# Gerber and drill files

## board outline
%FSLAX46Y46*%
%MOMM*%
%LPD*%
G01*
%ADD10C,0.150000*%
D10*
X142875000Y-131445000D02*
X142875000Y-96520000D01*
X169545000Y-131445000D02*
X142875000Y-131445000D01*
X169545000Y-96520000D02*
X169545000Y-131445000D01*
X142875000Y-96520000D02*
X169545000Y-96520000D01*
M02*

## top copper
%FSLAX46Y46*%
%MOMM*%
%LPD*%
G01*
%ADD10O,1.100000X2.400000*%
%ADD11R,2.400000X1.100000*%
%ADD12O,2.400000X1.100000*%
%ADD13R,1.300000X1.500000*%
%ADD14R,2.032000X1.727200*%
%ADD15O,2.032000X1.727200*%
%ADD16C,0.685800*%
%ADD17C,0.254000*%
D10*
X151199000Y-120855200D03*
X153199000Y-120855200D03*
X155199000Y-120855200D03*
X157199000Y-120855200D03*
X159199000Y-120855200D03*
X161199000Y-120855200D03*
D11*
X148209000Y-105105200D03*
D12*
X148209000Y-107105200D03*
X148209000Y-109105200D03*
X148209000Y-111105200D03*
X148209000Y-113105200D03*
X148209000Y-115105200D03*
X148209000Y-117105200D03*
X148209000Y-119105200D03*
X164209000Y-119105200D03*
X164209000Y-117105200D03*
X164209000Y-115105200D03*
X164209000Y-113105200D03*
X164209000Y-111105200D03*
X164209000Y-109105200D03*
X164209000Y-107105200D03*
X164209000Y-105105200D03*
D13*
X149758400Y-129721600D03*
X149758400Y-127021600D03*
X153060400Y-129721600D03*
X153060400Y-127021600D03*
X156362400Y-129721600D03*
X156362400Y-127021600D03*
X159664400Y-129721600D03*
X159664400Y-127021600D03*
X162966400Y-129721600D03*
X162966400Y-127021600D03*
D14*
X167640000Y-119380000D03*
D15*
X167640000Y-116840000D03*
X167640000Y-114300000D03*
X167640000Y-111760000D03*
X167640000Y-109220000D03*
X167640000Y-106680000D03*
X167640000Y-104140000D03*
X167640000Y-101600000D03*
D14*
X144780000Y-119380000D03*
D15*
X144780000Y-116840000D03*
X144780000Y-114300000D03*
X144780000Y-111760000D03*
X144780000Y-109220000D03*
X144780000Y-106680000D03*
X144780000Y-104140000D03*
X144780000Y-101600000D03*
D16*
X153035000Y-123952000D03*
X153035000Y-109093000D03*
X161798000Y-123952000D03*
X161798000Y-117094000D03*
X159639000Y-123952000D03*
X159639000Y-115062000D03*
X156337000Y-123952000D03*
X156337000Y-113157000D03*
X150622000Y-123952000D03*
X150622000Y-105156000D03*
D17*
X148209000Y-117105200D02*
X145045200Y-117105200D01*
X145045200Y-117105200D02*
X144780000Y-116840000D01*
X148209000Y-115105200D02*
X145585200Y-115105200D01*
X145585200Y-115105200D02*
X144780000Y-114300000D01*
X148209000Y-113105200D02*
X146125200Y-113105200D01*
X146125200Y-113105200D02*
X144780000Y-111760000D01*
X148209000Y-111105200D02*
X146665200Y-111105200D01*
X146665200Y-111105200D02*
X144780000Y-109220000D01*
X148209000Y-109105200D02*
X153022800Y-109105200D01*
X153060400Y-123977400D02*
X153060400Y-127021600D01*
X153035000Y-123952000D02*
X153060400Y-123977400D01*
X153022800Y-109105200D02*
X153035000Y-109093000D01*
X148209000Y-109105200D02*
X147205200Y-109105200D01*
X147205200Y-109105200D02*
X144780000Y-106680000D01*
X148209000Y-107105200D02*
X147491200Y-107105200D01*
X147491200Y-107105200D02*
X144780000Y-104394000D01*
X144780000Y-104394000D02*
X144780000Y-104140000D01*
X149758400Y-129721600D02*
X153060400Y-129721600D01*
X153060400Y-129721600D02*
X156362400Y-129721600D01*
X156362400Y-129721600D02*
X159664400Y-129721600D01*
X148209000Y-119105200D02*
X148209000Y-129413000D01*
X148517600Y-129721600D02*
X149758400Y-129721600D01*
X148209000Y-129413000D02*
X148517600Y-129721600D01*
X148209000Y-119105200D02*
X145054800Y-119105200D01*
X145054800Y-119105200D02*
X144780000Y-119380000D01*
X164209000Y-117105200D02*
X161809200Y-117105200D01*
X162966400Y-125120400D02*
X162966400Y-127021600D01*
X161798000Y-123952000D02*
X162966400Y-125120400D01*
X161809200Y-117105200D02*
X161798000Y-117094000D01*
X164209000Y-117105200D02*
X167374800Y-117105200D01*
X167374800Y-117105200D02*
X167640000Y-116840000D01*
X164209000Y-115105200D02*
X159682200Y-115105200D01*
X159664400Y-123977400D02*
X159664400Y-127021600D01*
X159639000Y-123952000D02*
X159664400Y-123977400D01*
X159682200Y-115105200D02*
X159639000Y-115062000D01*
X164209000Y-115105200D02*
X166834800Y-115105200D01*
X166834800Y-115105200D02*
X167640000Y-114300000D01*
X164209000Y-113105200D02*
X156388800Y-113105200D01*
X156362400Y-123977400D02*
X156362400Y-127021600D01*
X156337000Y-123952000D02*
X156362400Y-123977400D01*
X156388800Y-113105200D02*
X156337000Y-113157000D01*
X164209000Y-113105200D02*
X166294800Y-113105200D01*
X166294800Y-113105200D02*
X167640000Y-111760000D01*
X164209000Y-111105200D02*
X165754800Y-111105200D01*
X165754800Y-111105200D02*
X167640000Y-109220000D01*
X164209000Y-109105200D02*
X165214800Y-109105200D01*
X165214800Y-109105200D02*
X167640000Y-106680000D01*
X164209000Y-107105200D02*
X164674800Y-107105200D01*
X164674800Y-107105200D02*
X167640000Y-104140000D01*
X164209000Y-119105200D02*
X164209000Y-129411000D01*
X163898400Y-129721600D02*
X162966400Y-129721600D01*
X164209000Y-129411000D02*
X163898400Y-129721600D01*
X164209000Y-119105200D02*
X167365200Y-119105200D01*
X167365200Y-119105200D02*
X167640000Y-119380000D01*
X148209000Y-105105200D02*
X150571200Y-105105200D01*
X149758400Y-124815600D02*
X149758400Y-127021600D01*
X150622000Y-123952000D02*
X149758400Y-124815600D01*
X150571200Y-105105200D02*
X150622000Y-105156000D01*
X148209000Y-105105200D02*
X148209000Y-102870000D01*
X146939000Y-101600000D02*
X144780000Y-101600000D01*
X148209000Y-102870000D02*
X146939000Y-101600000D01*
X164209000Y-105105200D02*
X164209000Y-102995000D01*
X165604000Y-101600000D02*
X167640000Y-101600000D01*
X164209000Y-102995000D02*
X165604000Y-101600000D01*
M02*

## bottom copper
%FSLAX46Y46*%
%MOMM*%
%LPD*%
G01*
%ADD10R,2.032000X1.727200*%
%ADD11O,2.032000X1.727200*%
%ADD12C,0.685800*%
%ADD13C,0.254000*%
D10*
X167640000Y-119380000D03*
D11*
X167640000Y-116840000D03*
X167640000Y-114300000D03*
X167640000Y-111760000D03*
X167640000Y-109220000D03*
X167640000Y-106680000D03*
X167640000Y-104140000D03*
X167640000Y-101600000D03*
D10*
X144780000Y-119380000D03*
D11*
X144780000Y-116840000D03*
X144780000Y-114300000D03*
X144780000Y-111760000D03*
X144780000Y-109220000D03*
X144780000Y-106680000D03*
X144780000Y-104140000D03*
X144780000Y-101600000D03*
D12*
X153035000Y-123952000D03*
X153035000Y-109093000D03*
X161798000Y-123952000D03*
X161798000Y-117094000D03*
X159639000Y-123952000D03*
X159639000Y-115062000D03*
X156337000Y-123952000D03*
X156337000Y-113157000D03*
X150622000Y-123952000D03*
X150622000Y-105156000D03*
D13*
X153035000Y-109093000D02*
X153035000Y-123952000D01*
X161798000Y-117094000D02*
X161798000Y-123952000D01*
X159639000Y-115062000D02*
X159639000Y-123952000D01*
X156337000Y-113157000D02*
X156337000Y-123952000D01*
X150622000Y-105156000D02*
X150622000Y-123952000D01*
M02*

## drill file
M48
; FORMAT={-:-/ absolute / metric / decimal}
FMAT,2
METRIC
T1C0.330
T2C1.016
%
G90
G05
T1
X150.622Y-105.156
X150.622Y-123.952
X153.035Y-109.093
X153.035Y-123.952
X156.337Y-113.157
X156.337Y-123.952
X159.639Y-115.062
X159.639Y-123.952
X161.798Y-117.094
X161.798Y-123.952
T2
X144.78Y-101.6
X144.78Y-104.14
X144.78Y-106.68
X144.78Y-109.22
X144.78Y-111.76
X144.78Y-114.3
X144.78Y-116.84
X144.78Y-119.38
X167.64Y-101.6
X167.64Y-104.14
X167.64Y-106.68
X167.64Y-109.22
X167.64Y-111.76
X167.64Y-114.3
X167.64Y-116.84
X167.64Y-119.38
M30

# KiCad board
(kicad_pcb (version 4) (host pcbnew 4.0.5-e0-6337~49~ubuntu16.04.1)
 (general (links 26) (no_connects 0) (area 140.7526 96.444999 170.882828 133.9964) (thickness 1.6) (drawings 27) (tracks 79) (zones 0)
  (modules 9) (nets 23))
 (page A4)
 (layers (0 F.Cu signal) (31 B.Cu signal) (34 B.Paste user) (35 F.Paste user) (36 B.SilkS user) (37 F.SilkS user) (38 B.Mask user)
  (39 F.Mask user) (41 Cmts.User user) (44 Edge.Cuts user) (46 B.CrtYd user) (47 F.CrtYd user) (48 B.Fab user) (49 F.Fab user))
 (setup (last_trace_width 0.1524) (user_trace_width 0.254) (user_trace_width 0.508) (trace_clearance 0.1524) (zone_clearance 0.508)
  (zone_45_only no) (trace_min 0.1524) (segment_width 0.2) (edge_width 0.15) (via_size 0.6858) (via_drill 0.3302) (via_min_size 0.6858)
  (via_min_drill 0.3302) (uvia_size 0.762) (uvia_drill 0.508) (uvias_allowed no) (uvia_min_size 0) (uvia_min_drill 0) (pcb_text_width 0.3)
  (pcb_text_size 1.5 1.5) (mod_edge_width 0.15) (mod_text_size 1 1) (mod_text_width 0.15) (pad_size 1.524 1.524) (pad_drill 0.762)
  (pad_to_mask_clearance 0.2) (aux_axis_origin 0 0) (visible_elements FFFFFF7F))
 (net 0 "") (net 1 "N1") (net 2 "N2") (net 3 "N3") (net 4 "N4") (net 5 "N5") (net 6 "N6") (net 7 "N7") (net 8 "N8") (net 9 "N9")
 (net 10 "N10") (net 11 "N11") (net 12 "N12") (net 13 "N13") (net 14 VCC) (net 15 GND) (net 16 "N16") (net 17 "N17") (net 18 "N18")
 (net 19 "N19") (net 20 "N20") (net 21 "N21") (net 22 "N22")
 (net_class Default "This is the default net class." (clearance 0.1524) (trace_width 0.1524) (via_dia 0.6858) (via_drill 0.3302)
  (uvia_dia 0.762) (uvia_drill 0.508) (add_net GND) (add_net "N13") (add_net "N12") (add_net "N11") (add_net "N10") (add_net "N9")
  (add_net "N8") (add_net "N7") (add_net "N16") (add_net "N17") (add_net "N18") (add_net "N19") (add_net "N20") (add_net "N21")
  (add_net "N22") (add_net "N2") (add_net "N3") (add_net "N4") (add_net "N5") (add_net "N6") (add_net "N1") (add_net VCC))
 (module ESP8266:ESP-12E (layer F.Cu) (at 148.209 105.1052)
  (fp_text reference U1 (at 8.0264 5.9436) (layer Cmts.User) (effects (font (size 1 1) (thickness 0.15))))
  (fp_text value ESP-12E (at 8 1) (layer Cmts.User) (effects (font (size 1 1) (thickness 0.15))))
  (pad 9 smd oval (at 2.99 15.75 90) (size 2.4 1.1) (layers F.Cu F.Paste F.Mask) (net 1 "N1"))
  (pad 10 smd oval (at 4.99 15.75 90) (size 2.4 1.1) (layers F.Cu F.Paste F.Mask) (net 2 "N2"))
  (pad 11 smd oval (at 6.99 15.75 90) (size 2.4 1.1) (layers F.Cu F.Paste F.Mask) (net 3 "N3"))
  (pad 12 smd oval (at 8.99 15.75 90) (size 2.4 1.1) (layers F.Cu F.Paste F.Mask) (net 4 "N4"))
  (pad 13 smd oval (at 10.99 15.75 90) (size 2.4 1.1) (layers F.Cu F.Paste F.Mask) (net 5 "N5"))
  (pad 14 smd oval (at 12.99 15.75 90) (size 2.4 1.1) (layers F.Cu F.Paste F.Mask) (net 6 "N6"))
  (pad 1 smd rect (at 0 0) (size 2.4 1.1) (layers F.Cu F.Paste F.Mask) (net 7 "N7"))
  (pad 2 smd oval (at 0 2) (size 2.4 1.1) (layers F.Cu F.Paste F.Mask) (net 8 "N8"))
  (pad 3 smd oval (at 0 4) (size 2.4 1.1) (layers F.Cu F.Paste F.Mask) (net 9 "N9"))
  (pad 4 smd oval (at 0 6) (size 2.4 1.1) (layers F.Cu F.Paste F.Mask) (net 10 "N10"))
  (pad 5 smd oval (at 0 8) (size 2.4 1.1) (layers F.Cu F.Paste F.Mask) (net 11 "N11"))
  (pad 6 smd oval (at 0 10) (size 2.4 1.1) (layers F.Cu F.Paste F.Mask) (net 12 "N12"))
  (pad 7 smd oval (at 0 12) (size 2.4 1.1) (layers F.Cu F.Paste F.Mask) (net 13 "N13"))
  (pad 8 smd oval (at 0 14) (size 2.4 1.1) (layers F.Cu F.Paste F.Mask) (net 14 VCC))
  (pad 15 smd oval (at 16 14) (size 2.4 1.1) (layers F.Cu F.Paste F.Mask) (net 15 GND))
  (pad 16 smd oval (at 16 12) (size 2.4 1.1) (layers F.Cu F.Paste F.Mask) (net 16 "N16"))
  (pad 17 smd oval (at 16 10) (size 2.4 1.1) (layers F.Cu F.Paste F.Mask) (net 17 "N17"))
  (pad 18 smd oval (at 16 8) (size 2.4 1.1) (layers F.Cu F.Paste F.Mask) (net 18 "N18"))
  (pad 19 smd oval (at 16 6) (size 2.4 1.1) (layers F.Cu F.Paste F.Mask) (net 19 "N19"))
  (pad 20 smd oval (at 16 4) (size 2.4 1.1) (layers F.Cu F.Paste F.Mask) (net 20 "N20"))
  (pad 21 smd oval (at 16 2) (size 2.4 1.1) (layers F.Cu F.Paste F.Mask) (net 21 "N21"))
  (pad 22 smd oval (at 16 0) (size 2.4 1.1) (layers F.Cu F.Paste F.Mask) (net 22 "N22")))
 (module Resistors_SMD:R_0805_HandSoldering (layer F.Cu) (at 149.7584 128.3716 90)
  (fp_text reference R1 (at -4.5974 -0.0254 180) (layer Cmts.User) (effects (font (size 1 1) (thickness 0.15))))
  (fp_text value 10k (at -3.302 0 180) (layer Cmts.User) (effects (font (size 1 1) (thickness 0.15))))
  (pad 1 smd rect (at -1.35 0 90) (size 1.5 1.3) (layers F.Cu F.Paste F.Mask) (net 14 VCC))
  (pad 2 smd rect (at 1.35 0 90) (size 1.5 1.3) (layers F.Cu F.Paste F.Mask) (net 7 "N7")))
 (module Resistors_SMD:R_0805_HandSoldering (layer F.Cu) (at 153.0604 128.3716 90)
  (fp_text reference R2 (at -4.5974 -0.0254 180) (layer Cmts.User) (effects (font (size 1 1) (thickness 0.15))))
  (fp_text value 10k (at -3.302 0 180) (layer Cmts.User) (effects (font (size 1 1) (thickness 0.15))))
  (pad 1 smd rect (at -1.35 0 90) (size 1.5 1.3) (layers F.Cu F.Paste F.Mask) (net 14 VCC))
  (pad 2 smd rect (at 1.35 0 90) (size 1.5 1.3) (layers F.Cu F.Paste F.Mask) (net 9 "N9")))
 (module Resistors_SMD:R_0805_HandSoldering (layer F.Cu) (at 156.3624 128.3716 90)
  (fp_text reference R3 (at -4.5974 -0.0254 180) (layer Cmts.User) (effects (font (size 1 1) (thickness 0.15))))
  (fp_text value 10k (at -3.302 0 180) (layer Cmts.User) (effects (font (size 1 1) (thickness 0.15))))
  (pad 1 smd rect (at -1.35 0 90) (size 1.5 1.3) (layers F.Cu F.Paste F.Mask) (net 14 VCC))
  (pad 2 smd rect (at 1.35 0 90) (size 1.5 1.3) (layers F.Cu F.Paste F.Mask) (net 18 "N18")))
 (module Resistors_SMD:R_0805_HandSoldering (layer F.Cu) (at 159.6644 128.3716 90)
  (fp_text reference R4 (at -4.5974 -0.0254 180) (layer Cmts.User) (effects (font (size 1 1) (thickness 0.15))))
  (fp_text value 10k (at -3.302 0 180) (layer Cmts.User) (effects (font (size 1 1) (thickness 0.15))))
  (pad 1 smd rect (at -1.35 0 90) (size 1.5 1.3) (layers F.Cu F.Paste F.Mask) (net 14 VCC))
  (pad 2 smd rect (at 1.35 0 90) (size 1.5 1.3) (layers F.Cu F.Paste F.Mask) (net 17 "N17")))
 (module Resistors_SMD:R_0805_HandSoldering (layer F.Cu) (at 162.9664 128.3716 90)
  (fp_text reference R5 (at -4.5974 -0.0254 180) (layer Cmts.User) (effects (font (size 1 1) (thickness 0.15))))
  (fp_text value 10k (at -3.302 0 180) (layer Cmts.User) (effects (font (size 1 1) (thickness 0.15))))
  (pad 1 smd rect (at -1.35 0 90) (size 1.5 1.3) (layers F.Cu F.Paste F.Mask) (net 15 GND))
  (pad 2 smd rect (at 1.35 0 90) (size 1.5 1.3) (layers F.Cu F.Paste F.Mask) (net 16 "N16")))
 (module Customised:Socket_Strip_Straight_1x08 (layer F.Cu) (at 167.64 119.38 90)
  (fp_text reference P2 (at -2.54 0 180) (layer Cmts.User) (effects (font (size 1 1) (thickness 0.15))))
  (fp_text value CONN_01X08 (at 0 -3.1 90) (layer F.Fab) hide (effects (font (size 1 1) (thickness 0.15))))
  (pad 1 thru_hole rect (at 0 0 90) (size 1.7272 2.032) (drill 1.016) (layers *.Cu *.Mask) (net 15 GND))
  (pad 2 thru_hole oval (at 2.54 0 90) (size 1.7272 2.032) (drill 1.016) (layers *.Cu *.Mask) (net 16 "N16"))
  (pad 3 thru_hole oval (at 5.08 0 90) (size 1.7272 2.032) (drill 1.016) (layers *.Cu *.Mask) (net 17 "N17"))
  (pad 4 thru_hole oval (at 7.62 0 90) (size 1.7272 2.032) (drill 1.016) (layers *.Cu *.Mask) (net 18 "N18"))
  (pad 5 thru_hole oval (at 10.16 0 90) (size 1.7272 2.032) (drill 1.016) (layers *.Cu *.Mask) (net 19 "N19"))
  (pad 6 thru_hole oval (at 12.7 0 90) (size 1.7272 2.032) (drill 1.016) (layers *.Cu *.Mask) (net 20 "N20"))
  (pad 7 thru_hole oval (at 15.24 0 90) (size 1.7272 2.032) (drill 1.016) (layers *.Cu *.Mask) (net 21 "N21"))
  (pad 8 thru_hole oval (at 17.78 0 90) (size 1.7272 2.032) (drill 1.016) (layers *.Cu *.Mask) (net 22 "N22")))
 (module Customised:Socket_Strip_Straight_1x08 (layer F.Cu) (at 144.78 119.38 90)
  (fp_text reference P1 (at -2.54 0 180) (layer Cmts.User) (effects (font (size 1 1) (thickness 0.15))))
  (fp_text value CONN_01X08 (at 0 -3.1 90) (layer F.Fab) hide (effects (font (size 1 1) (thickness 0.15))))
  (pad 1 thru_hole rect (at 0 0 90) (size 1.7272 2.032) (drill 1.016) (layers *.Cu *.Mask) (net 14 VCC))
  (pad 2 thru_hole oval (at 2.54 0 90) (size 1.7272 2.032) (drill 1.016) (layers *.Cu *.Mask) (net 13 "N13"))
  (pad 3 thru_hole oval (at 5.08 0 90) (size 1.7272 2.032) (drill 1.016) (layers *.Cu *.Mask) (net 12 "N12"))
  (pad 4 thru_hole oval (at 7.62 0 90) (size 1.7272 2.032) (drill 1.016) (layers *.Cu *.Mask) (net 11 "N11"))
  (pad 5 thru_hole oval (at 10.16 0 90) (size 1.7272 2.032) (drill 1.016) (layers *.Cu *.Mask) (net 10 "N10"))
  (pad 6 thru_hole oval (at 12.7 0 90) (size 1.7272 2.032) (drill 1.016) (layers *.Cu *.Mask) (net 9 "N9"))
  (pad 7 thru_hole oval (at 15.24 0 90) (size 1.7272 2.032) (drill 1.016) (layers *.Cu *.Mask) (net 8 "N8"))
  (pad 8 thru_hole oval (at 17.78 0 90) (size 1.7272 2.032) (drill 1.016) (layers *.Cu *.Mask) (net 7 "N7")))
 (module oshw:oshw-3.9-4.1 (layer F.Cu) (at 167.005 128.27)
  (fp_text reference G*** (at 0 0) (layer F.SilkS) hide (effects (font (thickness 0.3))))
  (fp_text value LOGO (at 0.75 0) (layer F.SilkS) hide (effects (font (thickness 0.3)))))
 (gr_line (start 142.875 131.445) (end 142.875 96.52) (angle 90) (layer Edge.Cuts) (width 0.15))
 (gr_line (start 169.545 131.445) (end 142.875 131.445) (angle 90) (layer Edge.Cuts) (width 0.15))
 (gr_line (start 169.545 96.52) (end 169.545 131.445) (angle 90) (layer Edge.Cuts) (width 0.15))
 (gr_line (start 142.875 96.52) (end 169.545 96.52) (angle 90) (layer Edge.Cuts) (width 0.15))
 (segment (start 148.209 117.1052) (end 145.0452 117.1052) (width 0.254) (layer F.Cu) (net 13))
 (segment (start 145.0452 117.1052) (end 144.78 116.84) (width 0.254) (layer F.Cu) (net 13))
 (segment (start 148.209 115.1052) (end 145.5852 115.1052) (width 0.254) (layer F.Cu) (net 12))
 (segment (start 145.5852 115.1052) (end 144.78 114.3) (width 0.254) (layer F.Cu) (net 12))
 (segment (start 148.209 113.1052) (end 146.1252 113.1052) (width 0.254) (layer F.Cu) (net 11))
 (segment (start 146.1252 113.1052) (end 144.78 111.76) (width 0.254) (layer F.Cu) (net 11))
 (segment (start 148.209 111.1052) (end 146.6652 111.1052) (width 0.254) (layer F.Cu) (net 10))
 (segment (start 146.6652 111.1052) (end 144.78 109.22) (width 0.254) (layer F.Cu) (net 10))
 (segment (start 148.209 109.1052) (end 153.0228 109.1052) (width 0.254) (layer F.Cu) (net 9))
 (segment (start 153.0604 123.9774) (end 153.0604 127.0216) (width 0.254) (layer F.Cu) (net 9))
 (segment (start 153.035 123.952) (end 153.0604 123.9774) (width 0.254) (layer F.Cu) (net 9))
 (via (at 153.035 123.952) (size 0.6858) (drill 0.3302) (layers F.Cu B.Cu) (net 9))
 (segment (start 153.035 109.093) (end 153.035 123.952) (width 0.254) (layer B.Cu) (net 9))
 (via (at 153.035 109.093) (size 0.6858) (drill 0.3302) (layers F.Cu B.Cu) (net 9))
 (segment (start 153.0228 109.1052) (end 153.035 109.093) (width 0.254) (layer F.Cu) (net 9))
 (segment (start 148.209 109.1052) (end 147.2052 109.1052) (width 0.254) (layer F.Cu) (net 9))
 (segment (start 147.2052 109.1052) (end 144.78 106.68) (width 0.254) (layer F.Cu) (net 9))
 (segment (start 148.209 107.1052) (end 147.4912 107.1052) (width 0.254) (layer F.Cu) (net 8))
 (segment (start 147.4912 107.1052) (end 144.78 104.394) (width 0.254) (layer F.Cu) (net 8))
 (segment (start 144.78 104.394) (end 144.78 104.14) (width 0.254) (layer F.Cu) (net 8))
 (segment (start 149.7584 129.7216) (end 153.0604 129.7216) (width 0.254) (layer F.Cu) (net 14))
 (segment (start 153.0604 129.7216) (end 156.3624 129.7216) (width 0.254) (layer F.Cu) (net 14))
 (segment (start 156.3624 129.7216) (end 159.6644 129.7216) (width 0.254) (layer F.Cu) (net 14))
 (segment (start 148.209 119.1052) (end 148.209 129.413) (width 0.254) (layer F.Cu) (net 14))
 (segment (start 148.5176 129.7216) (end 149.7584 129.7216) (width 0.254) (layer F.Cu) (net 14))
 (segment (start 148.209 129.413) (end 148.5176 129.7216) (width 0.254) (layer F.Cu) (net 14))
 (segment (start 148.209 119.1052) (end 145.0548 119.1052) (width 0.254) (layer F.Cu) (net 14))
 (segment (start 145.0548 119.1052) (end 144.78 119.38) (width 0.254) (layer F.Cu) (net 14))
 (segment (start 164.209 117.1052) (end 161.8092 117.1052) (width 0.254) (layer F.Cu) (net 16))
 (segment (start 162.9664 125.1204) (end 162.9664 127.0216) (width 0.254) (layer F.Cu) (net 16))
 (segment (start 161.798 123.952) (end 162.9664 125.1204) (width 0.254) (layer F.Cu) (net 16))
 (via (at 161.798 123.952) (size 0.6858) (drill 0.3302) (layers F.Cu B.Cu) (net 16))
 (segment (start 161.798 117.094) (end 161.798 123.952) (width 0.254) (layer B.Cu) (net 16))
 (via (at 161.798 117.094) (size 0.6858) (drill 0.3302) (layers F.Cu B.Cu) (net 16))
 (segment (start 161.8092 117.1052) (end 161.798 117.094) (width 0.254) (layer F.Cu) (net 16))
 (segment (start 164.209 117.1052) (end 167.3748 117.1052) (width 0.254) (layer F.Cu) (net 16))
 (segment (start 167.3748 117.1052) (end 167.64 116.84) (width 0.254) (layer F.Cu) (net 16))
 (segment (start 164.209 115.1052) (end 159.6822 115.1052) (width 0.254) (layer F.Cu) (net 17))
 (segment (start 159.6644 123.9774) (end 159.6644 127.0216) (width 0.254) (layer F.Cu) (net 17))
 (segment (start 159.639 123.952) (end 159.6644 123.9774) (width 0.254) (layer F.Cu) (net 17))
 (via (at 159.639 123.952) (size 0.6858) (drill 0.3302) (layers F.Cu B.Cu) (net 17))
 (segment (start 159.639 115.062) (end 159.639 123.952) (width 0.254) (layer B.Cu) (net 17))
 (via (at 159.639 115.062) (size 0.6858) (drill 0.3302) (layers F.Cu B.Cu) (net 17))
 (segment (start 159.6822 115.1052) (end 159.639 115.062) (width 0.254) (layer F.Cu) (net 17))
 (segment (start 164.209 115.1052) (end 166.8348 115.1052) (width 0.254) (layer F.Cu) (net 17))
 (segment (start 166.8348 115.1052) (end 167.64 114.3) (width 0.254) (layer F.Cu) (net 17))
 (segment (start 164.209 113.1052) (end 156.3888 113.1052) (width 0.254) (layer F.Cu) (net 18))
 (segment (start 156.3624 123.9774) (end 156.3624 127.0216) (width 0.254) (layer F.Cu) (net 18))
 (segment (start 156.337 123.952) (end 156.3624 123.9774) (width 0.254) (layer F.Cu) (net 18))
 (via (at 156.337 123.952) (size 0.6858) (drill 0.3302) (layers F.Cu B.Cu) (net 18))
 (segment (start 156.337 113.157) (end 156.337 123.952) (width 0.254) (layer B.Cu) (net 18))
 (via (at 156.337 113.157) (size 0.6858) (drill 0.3302) (layers F.Cu B.Cu) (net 18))
 (segment (start 156.3888 113.1052) (end 156.337 113.157) (width 0.254) (layer F.Cu) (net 18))
 (segment (start 164.209 113.1052) (end 166.2948 113.1052) (width 0.254) (layer F.Cu) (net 18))
 (segment (start 166.2948 113.1052) (end 167.64 111.76) (width 0.254) (layer F.Cu) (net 18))
 (segment (start 164.209 111.1052) (end 165.7548 111.1052) (width 0.254) (layer F.Cu) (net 19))
 (segment (start 165.7548 111.1052) (end 167.64 109.22) (width 0.254) (layer F.Cu) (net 19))
 (segment (start 164.209 109.1052) (end 165.2148 109.1052) (width 0.254) (layer F.Cu) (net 20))
 (segment (start 165.2148 109.1052) (end 167.64 106.68) (width 0.254) (layer F.Cu) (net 20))
 (segment (start 164.209 107.1052) (end 164.6748 107.1052) (width 0.254) (layer F.Cu) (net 21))
 (segment (start 164.6748 107.1052) (end 167.64 104.14) (width 0.254) (layer F.Cu) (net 21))
 (segment (start 164.209 119.1052) (end 164.209 129.411) (width 0.254) (layer F.Cu) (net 15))
 (segment (start 163.8984 129.7216) (end 162.9664 129.7216) (width 0.254) (layer F.Cu) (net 15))
 (segment (start 164.209 129.411) (end 163.8984 129.7216) (width 0.254) (layer F.Cu) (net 15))
 (segment (start 164.209 119.1052) (end 167.3652 119.1052) (width 0.254) (layer F.Cu) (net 15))
 (segment (start 167.3652 119.1052) (end 167.64 119.38) (width 0.254) (layer F.Cu) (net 15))
 (segment (start 148.209 105.1052) (end 150.5712 105.1052) (width 0.254) (layer F.Cu) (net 7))
 (segment (start 149.7584 124.8156) (end 149.7584 127.0216) (width 0.254) (layer F.Cu) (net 7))
 (segment (start 150.622 123.952) (end 149.7584 124.8156) (width 0.254) (layer F.Cu) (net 7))
 (via (at 150.622 123.952) (size 0.6858) (drill 0.3302) (layers F.Cu B.Cu) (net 7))
 (segment (start 150.622 105.156) (end 150.622 123.952) (width 0.254) (layer B.Cu) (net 7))
 (via (at 150.622 105.156) (size 0.6858) (drill 0.3302) (layers F.Cu B.Cu) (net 7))
 (segment (start 150.5712 105.1052) (end 150.622 105.156) (width 0.254) (layer F.Cu) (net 7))
 (segment (start 148.209 105.1052) (end 148.209 102.87) (width 0.254) (layer F.Cu) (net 7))
 (segment (start 146.939 101.6) (end 144.78 101.6) (width 0.254) (layer F.Cu) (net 7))
 (segment (start 148.209 102.87) (end 146.939 101.6) (width 0.254) (layer F.Cu) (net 7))
 (segment (start 164.209 105.1052) (end 164.209 102.995) (width 0.254) (layer F.Cu) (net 22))
 (segment (start 165.604 101.6) (end 167.64 101.6) (width 0.254) (layer F.Cu) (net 22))
 (segment (start 164.209 102.995) (end 165.604 101.6) (width 0.254) (layer F.Cu) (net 22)))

